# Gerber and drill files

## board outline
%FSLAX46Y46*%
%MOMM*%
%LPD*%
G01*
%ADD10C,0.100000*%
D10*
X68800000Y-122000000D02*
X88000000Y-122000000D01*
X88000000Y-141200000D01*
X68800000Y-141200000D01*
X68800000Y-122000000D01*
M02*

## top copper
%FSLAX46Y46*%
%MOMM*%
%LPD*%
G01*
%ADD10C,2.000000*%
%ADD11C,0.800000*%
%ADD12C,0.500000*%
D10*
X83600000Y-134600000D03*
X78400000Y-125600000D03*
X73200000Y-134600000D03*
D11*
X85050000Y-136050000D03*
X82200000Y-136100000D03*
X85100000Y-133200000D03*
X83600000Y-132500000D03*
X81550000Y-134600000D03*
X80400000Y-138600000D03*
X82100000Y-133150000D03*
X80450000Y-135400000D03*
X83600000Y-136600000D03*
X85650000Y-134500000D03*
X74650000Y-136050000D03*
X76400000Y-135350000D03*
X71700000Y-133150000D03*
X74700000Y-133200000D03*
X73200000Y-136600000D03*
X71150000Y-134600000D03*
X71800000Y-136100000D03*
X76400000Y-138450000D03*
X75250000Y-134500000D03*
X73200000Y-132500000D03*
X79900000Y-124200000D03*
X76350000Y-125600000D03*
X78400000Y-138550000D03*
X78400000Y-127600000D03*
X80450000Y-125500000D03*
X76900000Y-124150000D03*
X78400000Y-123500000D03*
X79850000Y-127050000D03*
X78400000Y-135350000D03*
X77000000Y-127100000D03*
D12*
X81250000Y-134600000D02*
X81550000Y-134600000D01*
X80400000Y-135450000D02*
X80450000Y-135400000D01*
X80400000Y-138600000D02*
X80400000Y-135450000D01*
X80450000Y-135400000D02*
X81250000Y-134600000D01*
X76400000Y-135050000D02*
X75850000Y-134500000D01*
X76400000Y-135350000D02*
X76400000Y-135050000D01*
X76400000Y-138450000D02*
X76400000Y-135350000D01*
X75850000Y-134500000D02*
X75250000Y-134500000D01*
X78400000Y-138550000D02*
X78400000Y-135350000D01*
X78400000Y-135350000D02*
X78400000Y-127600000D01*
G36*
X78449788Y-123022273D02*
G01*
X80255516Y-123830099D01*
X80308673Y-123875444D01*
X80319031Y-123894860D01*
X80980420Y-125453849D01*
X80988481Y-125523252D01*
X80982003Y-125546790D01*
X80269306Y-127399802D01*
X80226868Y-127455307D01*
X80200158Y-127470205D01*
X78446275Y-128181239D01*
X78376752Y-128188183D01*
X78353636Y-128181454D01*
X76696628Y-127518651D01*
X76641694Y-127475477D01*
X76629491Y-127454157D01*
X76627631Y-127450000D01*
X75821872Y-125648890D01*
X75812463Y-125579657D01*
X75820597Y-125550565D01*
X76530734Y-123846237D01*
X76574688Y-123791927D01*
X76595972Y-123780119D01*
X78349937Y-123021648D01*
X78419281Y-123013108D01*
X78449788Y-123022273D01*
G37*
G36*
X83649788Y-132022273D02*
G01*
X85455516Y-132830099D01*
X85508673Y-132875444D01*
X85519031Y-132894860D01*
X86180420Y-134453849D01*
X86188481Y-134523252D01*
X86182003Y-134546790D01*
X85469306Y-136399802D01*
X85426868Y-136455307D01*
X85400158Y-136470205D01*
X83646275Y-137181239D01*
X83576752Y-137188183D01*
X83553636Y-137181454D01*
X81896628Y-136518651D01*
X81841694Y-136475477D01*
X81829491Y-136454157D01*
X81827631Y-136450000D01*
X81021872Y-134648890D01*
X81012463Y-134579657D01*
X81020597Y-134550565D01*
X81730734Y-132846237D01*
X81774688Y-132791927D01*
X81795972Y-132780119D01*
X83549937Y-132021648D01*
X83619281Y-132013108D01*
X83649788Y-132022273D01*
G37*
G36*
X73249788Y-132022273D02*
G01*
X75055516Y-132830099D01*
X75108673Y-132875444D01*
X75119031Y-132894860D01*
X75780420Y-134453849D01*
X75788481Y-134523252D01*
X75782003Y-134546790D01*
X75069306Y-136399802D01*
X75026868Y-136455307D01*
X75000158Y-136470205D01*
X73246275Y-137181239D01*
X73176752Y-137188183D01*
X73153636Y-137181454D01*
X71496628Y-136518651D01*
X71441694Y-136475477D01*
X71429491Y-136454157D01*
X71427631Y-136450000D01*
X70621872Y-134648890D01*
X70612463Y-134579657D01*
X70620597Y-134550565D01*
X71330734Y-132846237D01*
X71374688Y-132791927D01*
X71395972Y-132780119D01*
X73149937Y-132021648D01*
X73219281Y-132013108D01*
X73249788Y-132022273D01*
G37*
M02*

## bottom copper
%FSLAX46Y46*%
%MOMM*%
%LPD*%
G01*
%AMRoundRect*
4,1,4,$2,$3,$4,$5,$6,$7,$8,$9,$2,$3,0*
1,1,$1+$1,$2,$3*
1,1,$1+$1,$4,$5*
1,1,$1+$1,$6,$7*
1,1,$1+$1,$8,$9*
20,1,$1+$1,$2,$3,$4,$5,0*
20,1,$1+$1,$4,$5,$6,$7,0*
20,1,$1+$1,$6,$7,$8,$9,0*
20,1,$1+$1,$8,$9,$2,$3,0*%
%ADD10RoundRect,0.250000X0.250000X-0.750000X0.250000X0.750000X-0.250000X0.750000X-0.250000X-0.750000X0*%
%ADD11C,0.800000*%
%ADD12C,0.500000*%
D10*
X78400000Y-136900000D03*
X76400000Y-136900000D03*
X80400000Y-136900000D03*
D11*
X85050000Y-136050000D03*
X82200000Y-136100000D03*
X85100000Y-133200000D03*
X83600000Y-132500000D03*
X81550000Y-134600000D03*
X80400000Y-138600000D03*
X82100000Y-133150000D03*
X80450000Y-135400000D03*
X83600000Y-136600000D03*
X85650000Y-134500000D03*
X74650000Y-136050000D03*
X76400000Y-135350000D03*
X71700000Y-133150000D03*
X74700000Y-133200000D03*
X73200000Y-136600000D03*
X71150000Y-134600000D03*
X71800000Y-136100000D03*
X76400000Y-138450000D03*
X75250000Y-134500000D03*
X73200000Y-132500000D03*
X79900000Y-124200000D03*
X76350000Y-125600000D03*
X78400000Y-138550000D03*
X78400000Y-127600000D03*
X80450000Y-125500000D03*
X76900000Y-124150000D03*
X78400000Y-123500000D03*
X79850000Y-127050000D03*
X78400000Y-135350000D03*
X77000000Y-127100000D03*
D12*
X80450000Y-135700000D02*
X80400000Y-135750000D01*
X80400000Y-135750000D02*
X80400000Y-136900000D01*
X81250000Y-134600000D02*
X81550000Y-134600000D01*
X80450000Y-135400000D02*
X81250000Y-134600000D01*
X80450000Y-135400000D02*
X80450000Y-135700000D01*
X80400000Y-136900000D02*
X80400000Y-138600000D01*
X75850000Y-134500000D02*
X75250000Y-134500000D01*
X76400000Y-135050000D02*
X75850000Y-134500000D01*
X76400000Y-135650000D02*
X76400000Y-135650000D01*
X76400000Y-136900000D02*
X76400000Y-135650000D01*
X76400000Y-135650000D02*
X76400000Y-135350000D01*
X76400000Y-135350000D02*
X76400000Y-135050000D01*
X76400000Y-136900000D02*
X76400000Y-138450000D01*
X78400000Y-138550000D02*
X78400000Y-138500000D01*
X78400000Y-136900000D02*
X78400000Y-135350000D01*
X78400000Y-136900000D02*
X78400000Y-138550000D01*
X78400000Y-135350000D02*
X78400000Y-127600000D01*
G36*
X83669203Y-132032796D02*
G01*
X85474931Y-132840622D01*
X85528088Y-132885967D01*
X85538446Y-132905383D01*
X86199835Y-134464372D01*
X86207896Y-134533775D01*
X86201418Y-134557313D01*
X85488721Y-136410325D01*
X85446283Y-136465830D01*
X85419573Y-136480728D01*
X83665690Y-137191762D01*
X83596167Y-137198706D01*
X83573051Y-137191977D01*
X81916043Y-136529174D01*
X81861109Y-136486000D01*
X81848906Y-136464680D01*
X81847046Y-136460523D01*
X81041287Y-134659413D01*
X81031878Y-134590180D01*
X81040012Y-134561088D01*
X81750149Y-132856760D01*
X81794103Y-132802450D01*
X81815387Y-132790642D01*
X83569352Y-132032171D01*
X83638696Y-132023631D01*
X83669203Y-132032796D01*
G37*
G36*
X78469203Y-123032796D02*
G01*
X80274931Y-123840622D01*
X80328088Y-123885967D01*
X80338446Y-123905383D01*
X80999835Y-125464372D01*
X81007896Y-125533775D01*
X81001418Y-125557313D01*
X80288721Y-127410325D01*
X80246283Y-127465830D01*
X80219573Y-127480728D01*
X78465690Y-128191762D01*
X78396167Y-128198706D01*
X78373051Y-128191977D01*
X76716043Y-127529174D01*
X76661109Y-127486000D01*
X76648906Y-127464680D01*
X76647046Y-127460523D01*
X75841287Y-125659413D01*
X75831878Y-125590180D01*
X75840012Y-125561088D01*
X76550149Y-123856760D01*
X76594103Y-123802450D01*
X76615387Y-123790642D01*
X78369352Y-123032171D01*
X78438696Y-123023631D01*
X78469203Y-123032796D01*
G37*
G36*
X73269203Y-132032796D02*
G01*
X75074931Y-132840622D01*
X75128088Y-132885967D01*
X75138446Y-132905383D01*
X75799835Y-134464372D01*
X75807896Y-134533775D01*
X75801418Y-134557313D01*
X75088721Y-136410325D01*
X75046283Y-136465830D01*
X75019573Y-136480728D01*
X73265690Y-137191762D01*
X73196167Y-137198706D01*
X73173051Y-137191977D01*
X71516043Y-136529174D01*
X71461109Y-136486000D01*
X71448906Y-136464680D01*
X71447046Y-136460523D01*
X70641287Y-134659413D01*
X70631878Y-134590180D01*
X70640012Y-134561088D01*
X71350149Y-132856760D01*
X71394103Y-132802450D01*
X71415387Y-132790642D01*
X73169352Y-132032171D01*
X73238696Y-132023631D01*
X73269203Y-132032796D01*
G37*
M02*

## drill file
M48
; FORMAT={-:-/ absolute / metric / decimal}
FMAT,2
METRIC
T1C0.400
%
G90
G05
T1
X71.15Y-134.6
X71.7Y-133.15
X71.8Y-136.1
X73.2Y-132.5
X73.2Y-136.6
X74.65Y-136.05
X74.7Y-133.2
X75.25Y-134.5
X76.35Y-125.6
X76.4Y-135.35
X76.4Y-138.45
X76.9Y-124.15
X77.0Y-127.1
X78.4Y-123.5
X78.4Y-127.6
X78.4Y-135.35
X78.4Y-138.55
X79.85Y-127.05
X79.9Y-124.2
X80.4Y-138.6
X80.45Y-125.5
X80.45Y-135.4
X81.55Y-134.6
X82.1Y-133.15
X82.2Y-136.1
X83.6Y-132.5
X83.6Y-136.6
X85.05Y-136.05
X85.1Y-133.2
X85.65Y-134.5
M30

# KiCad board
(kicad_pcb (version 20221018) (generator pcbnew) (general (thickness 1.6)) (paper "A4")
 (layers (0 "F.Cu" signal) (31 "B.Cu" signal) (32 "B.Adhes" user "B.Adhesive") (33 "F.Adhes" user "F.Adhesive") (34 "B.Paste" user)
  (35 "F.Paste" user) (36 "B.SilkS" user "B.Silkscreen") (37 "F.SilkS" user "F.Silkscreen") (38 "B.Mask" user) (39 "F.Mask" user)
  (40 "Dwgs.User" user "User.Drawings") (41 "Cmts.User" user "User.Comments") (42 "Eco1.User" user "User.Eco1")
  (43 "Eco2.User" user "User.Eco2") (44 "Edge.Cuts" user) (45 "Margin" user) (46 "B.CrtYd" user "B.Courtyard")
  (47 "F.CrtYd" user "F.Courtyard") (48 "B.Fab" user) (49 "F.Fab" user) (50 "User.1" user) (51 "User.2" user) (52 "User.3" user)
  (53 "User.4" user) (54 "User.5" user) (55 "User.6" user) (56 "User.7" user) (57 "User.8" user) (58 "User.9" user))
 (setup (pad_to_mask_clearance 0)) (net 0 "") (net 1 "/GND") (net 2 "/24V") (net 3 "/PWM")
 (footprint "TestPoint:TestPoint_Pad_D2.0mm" (layer "F.Cu") (at 83.6 134.6)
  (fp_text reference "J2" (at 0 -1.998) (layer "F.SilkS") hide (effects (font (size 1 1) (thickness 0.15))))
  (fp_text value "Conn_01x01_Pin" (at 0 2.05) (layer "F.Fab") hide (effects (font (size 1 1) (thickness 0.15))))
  (pad "1" smd circle (at 0 0) (size 2 2) (layers "F.Cu" "F.Paste" "F.Mask") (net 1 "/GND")))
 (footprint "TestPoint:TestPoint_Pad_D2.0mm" (layer "F.Cu") (at 78.4 125.6)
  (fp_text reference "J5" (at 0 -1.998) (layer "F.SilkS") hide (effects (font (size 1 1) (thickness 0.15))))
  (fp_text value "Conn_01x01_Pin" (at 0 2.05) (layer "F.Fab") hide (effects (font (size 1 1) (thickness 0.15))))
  (pad "1" smd circle (at 0 0) (size 2 2) (layers "F.Cu" "F.Paste" "F.Mask") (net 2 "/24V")))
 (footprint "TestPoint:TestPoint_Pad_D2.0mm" (layer "F.Cu") (at 73.2 134.6)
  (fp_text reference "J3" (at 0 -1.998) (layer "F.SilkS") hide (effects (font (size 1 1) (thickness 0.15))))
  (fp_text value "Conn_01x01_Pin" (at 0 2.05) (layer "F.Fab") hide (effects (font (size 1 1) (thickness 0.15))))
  (pad "1" smd circle (at 0 0) (size 2 2) (layers "F.Cu" "F.Paste" "F.Mask") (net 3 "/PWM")))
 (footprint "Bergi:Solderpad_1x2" (layer "B.Cu") (at 78.4 136.9 90)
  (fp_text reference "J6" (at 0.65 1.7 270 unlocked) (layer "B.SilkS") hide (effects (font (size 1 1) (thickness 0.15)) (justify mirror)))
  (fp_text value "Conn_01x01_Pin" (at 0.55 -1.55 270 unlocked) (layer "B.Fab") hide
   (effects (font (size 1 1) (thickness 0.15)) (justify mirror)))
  (pad "1" smd roundrect (at 0 0 90) (size 2 1) (layers "B.Cu" "B.Mask") (roundrect_rratio 0.25) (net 2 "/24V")))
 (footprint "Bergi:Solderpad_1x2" (layer "B.Cu") (at 76.4 136.9 90)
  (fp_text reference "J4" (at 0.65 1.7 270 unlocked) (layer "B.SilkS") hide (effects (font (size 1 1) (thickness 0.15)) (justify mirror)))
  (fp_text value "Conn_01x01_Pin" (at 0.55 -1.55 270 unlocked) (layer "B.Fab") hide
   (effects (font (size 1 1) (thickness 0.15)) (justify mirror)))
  (pad "1" smd roundrect (at 0 0 90) (size 2 1) (layers "B.Cu" "B.Mask") (roundrect_rratio 0.25) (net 3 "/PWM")))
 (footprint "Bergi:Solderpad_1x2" (layer "B.Cu") (at 80.4 136.9 90)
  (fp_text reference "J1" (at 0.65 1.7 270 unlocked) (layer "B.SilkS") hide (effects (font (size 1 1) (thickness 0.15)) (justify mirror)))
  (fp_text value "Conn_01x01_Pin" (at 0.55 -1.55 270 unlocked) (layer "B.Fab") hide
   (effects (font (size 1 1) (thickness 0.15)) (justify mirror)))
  (pad "1" smd roundrect (at 0 0 90) (size 2 1) (layers "B.Cu" "B.Mask") (roundrect_rratio 0.25) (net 1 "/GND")))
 (gr_rect (start 68.8 122) (end 88 141.2) (stroke (width 0.1) (type default)) (fill none) (layer "Edge.Cuts"))
 (segment (start 81.25 134.6) (end 81.55 134.6) (width 0.5) (layer "F.Cu") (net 1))
 (segment (start 80.4 135.45) (end 80.45 135.4) (width 0.5) (layer "F.Cu") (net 1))
 (segment (start 80.4 138.6) (end 80.4 135.45) (width 0.5) (layer "F.Cu") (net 1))
 (segment (start 80.45 135.4) (end 81.25 134.6) (width 0.5) (layer "F.Cu") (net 1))
 (via (at 85.05 136.05) (size 0.8) (drill 0.4) (layers "F.Cu" "B.Cu") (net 1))
 (via (at 82.2 136.1) (size 0.8) (drill 0.4) (layers "F.Cu" "B.Cu") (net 1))
 (via (at 85.1 133.2) (size 0.8) (drill 0.4) (layers "F.Cu" "B.Cu") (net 1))
 (via (at 83.6 132.5) (size 0.8) (drill 0.4) (layers "F.Cu" "B.Cu") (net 1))
 (via (at 81.55 134.6) (size 0.8) (drill 0.4) (layers "F.Cu" "B.Cu") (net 1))
 (via (at 80.4 138.6) (size 0.8) (drill 0.4) (layers "F.Cu" "B.Cu") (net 1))
 (via (at 82.1 133.15) (size 0.8) (drill 0.4) (layers "F.Cu" "B.Cu") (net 1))
 (via (at 80.45 135.4) (size 0.8) (drill 0.4) (layers "F.Cu" "B.Cu") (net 1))
 (via (at 83.6 136.6) (size 0.8) (drill 0.4) (layers "F.Cu" "B.Cu") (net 1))
 (via (at 85.65 134.5) (size 0.8) (drill 0.4) (layers "F.Cu" "B.Cu") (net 1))
 (segment (start 80.45 135.7) (end 80.4 135.75) (width 0.5) (layer "B.Cu") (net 1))
 (segment (start 80.4 135.75) (end 80.4 136.9) (width 0.5) (layer "B.Cu") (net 1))
 (segment (start 81.25 134.6) (end 81.55 134.6) (width 0.5) (layer "B.Cu") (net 1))
 (segment (start 80.45 135.4) (end 81.25 134.6) (width 0.5) (layer "B.Cu") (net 1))
 (segment (start 80.45 135.4) (end 80.45 135.7) (width 0.5) (layer "B.Cu") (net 1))
 (segment (start 80.4 136.9) (end 80.4 138.6) (width 0.5) (layer "B.Cu") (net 1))
 (segment (start 76.4 135.05) (end 75.85 134.5) (width 0.5) (layer "F.Cu") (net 3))
 (segment (start 76.4 135.35) (end 76.4 135.05) (width 0.5) (layer "F.Cu") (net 3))
 (segment (start 76.4 138.45) (end 76.4 135.35) (width 0.5) (layer "F.Cu") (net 3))
 (segment (start 75.85 134.5) (end 75.25 134.5) (width 0.5) (layer "F.Cu") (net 3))
 (via (at 74.65 136.05) (size 0.8) (drill 0.4) (layers "F.Cu" "B.Cu") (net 3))
 (via (at 76.4 135.35) (size 0.8) (drill 0.4) (layers "F.Cu" "B.Cu") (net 3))
 (via (at 71.7 133.15) (size 0.8) (drill 0.4) (layers "F.Cu" "B.Cu") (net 3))
 (via (at 74.7 133.2) (size 0.8) (drill 0.4) (layers "F.Cu" "B.Cu") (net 3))
 (via (at 73.2 136.6) (size 0.8) (drill 0.4) (layers "F.Cu" "B.Cu") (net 3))
 (via (at 71.15 134.6) (size 0.8) (drill 0.4) (layers "F.Cu" "B.Cu") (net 3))
 (via (at 71.8 136.1) (size 0.8) (drill 0.4) (layers "F.Cu" "B.Cu") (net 3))
 (via (at 76.4 138.45) (size 0.8) (drill 0.4) (layers "F.Cu" "B.Cu") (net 3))
 (via (at 75.25 134.5) (size 0.8) (drill 0.4) (layers "F.Cu" "B.Cu") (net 3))
 (via (at 73.2 132.5) (size 0.8) (drill 0.4) (layers "F.Cu" "B.Cu") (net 3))
 (segment (start 75.85 134.5) (end 75.25 134.5) (width 0.5) (layer "B.Cu") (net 3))
 (segment (start 76.4 135.05) (end 75.85 134.5) (width 0.5) (layer "B.Cu") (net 3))
 (segment (start 76.4 135.65) (end 76.4 135.65) (width 0.5) (layer "B.Cu") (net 3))
 (segment (start 76.4 136.9) (end 76.4 135.65) (width 0.5) (layer "B.Cu") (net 3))
 (segment (start 76.4 135.65) (end 76.4 135.35) (width 0.5) (layer "B.Cu") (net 3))
 (segment (start 76.4 135.35) (end 76.4 135.05) (width 0.5) (layer "B.Cu") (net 3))
 (segment (start 76.4 136.9) (end 76.4 138.45) (width 0.5) (layer "B.Cu") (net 3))
 (segment (start 78.4 138.55) (end 78.4 135.35) (width 0.5) (layer "F.Cu") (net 2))
 (segment (start 78.4 135.35) (end 78.4 127.6) (width 0.5) (layer "F.Cu") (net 2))
 (via (at 79.9 124.2) (size 0.8) (drill 0.4) (layers "F.Cu" "B.Cu") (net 2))
 (via (at 76.35 125.6) (size 0.8) (drill 0.4) (layers "F.Cu" "B.Cu") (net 2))
 (via (at 78.4 138.55) (size 0.8) (drill 0.4) (layers "F.Cu" "B.Cu") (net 2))
 (via (at 78.4 127.6) (size 0.8) (drill 0.4) (layers "F.Cu" "B.Cu") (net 2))
 (via (at 80.45 125.5) (size 0.8) (drill 0.4) (layers "F.Cu" "B.Cu") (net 2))
 (via (at 76.9 124.15) (size 0.8) (drill 0.4) (layers "F.Cu" "B.Cu") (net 2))
 (via (at 78.4 123.5) (size 0.8) (drill 0.4) (layers "F.Cu" "B.Cu") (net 2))
 (via (at 79.85 127.05) (size 0.8) (drill 0.4) (layers "F.Cu" "B.Cu") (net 2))
 (via (at 78.4 135.35) (size 0.8) (drill 0.4) (layers "F.Cu" "B.Cu") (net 2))
 (via (at 77 127.1) (size 0.8) (drill 0.4) (layers "F.Cu" "B.Cu") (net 2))
 (segment (start 78.4 138.55) (end 78.4 138.5) (width 0.5) (layer "B.Cu") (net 2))
 (segment (start 78.4 136.9) (end 78.4 135.35) (width 0.5) (layer "B.Cu") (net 2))
 (segment (start 78.4 136.9) (end 78.4 138.55) (width 0.5) (layer "B.Cu") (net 2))
 (segment (start 78.4 135.35) (end 78.4 127.6) (width 0.5) (layer "B.Cu") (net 2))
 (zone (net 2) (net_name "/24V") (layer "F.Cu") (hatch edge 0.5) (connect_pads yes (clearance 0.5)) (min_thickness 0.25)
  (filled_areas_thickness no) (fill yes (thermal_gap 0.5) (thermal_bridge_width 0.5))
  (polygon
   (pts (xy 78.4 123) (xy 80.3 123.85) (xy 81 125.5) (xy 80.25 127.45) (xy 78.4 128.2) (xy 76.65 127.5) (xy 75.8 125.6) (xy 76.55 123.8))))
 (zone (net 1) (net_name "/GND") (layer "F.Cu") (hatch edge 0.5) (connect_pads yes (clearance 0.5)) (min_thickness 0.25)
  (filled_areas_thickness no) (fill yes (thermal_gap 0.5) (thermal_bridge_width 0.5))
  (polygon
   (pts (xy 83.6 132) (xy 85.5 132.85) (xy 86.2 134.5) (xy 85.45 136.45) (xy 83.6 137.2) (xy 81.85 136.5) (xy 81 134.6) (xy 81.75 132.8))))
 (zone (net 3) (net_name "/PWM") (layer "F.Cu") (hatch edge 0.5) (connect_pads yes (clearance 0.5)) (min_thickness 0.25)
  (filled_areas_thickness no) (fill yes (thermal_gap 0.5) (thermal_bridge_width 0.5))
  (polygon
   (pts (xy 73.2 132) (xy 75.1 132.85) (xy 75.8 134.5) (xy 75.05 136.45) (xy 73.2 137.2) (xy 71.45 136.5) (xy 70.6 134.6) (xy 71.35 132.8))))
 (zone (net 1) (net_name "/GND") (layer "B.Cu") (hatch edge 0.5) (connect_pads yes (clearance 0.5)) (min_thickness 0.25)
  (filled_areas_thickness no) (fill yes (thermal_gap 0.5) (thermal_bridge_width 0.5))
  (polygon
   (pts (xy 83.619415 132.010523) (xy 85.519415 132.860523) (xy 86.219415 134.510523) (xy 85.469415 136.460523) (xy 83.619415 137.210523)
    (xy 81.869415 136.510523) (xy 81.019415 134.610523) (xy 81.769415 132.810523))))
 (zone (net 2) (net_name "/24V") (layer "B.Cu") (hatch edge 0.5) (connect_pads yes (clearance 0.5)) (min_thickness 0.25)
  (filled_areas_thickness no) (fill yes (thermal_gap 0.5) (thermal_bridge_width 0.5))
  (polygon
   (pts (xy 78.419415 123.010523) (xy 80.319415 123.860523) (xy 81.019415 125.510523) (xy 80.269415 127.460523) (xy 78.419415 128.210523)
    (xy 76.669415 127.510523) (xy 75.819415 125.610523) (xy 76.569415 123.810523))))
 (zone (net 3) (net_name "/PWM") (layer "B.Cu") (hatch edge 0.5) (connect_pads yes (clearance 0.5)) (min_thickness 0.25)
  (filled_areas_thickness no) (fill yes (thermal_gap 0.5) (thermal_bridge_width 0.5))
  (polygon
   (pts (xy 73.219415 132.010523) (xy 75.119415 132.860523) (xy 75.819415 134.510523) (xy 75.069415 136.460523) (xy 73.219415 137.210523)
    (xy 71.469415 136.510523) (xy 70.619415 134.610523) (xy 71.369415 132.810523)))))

